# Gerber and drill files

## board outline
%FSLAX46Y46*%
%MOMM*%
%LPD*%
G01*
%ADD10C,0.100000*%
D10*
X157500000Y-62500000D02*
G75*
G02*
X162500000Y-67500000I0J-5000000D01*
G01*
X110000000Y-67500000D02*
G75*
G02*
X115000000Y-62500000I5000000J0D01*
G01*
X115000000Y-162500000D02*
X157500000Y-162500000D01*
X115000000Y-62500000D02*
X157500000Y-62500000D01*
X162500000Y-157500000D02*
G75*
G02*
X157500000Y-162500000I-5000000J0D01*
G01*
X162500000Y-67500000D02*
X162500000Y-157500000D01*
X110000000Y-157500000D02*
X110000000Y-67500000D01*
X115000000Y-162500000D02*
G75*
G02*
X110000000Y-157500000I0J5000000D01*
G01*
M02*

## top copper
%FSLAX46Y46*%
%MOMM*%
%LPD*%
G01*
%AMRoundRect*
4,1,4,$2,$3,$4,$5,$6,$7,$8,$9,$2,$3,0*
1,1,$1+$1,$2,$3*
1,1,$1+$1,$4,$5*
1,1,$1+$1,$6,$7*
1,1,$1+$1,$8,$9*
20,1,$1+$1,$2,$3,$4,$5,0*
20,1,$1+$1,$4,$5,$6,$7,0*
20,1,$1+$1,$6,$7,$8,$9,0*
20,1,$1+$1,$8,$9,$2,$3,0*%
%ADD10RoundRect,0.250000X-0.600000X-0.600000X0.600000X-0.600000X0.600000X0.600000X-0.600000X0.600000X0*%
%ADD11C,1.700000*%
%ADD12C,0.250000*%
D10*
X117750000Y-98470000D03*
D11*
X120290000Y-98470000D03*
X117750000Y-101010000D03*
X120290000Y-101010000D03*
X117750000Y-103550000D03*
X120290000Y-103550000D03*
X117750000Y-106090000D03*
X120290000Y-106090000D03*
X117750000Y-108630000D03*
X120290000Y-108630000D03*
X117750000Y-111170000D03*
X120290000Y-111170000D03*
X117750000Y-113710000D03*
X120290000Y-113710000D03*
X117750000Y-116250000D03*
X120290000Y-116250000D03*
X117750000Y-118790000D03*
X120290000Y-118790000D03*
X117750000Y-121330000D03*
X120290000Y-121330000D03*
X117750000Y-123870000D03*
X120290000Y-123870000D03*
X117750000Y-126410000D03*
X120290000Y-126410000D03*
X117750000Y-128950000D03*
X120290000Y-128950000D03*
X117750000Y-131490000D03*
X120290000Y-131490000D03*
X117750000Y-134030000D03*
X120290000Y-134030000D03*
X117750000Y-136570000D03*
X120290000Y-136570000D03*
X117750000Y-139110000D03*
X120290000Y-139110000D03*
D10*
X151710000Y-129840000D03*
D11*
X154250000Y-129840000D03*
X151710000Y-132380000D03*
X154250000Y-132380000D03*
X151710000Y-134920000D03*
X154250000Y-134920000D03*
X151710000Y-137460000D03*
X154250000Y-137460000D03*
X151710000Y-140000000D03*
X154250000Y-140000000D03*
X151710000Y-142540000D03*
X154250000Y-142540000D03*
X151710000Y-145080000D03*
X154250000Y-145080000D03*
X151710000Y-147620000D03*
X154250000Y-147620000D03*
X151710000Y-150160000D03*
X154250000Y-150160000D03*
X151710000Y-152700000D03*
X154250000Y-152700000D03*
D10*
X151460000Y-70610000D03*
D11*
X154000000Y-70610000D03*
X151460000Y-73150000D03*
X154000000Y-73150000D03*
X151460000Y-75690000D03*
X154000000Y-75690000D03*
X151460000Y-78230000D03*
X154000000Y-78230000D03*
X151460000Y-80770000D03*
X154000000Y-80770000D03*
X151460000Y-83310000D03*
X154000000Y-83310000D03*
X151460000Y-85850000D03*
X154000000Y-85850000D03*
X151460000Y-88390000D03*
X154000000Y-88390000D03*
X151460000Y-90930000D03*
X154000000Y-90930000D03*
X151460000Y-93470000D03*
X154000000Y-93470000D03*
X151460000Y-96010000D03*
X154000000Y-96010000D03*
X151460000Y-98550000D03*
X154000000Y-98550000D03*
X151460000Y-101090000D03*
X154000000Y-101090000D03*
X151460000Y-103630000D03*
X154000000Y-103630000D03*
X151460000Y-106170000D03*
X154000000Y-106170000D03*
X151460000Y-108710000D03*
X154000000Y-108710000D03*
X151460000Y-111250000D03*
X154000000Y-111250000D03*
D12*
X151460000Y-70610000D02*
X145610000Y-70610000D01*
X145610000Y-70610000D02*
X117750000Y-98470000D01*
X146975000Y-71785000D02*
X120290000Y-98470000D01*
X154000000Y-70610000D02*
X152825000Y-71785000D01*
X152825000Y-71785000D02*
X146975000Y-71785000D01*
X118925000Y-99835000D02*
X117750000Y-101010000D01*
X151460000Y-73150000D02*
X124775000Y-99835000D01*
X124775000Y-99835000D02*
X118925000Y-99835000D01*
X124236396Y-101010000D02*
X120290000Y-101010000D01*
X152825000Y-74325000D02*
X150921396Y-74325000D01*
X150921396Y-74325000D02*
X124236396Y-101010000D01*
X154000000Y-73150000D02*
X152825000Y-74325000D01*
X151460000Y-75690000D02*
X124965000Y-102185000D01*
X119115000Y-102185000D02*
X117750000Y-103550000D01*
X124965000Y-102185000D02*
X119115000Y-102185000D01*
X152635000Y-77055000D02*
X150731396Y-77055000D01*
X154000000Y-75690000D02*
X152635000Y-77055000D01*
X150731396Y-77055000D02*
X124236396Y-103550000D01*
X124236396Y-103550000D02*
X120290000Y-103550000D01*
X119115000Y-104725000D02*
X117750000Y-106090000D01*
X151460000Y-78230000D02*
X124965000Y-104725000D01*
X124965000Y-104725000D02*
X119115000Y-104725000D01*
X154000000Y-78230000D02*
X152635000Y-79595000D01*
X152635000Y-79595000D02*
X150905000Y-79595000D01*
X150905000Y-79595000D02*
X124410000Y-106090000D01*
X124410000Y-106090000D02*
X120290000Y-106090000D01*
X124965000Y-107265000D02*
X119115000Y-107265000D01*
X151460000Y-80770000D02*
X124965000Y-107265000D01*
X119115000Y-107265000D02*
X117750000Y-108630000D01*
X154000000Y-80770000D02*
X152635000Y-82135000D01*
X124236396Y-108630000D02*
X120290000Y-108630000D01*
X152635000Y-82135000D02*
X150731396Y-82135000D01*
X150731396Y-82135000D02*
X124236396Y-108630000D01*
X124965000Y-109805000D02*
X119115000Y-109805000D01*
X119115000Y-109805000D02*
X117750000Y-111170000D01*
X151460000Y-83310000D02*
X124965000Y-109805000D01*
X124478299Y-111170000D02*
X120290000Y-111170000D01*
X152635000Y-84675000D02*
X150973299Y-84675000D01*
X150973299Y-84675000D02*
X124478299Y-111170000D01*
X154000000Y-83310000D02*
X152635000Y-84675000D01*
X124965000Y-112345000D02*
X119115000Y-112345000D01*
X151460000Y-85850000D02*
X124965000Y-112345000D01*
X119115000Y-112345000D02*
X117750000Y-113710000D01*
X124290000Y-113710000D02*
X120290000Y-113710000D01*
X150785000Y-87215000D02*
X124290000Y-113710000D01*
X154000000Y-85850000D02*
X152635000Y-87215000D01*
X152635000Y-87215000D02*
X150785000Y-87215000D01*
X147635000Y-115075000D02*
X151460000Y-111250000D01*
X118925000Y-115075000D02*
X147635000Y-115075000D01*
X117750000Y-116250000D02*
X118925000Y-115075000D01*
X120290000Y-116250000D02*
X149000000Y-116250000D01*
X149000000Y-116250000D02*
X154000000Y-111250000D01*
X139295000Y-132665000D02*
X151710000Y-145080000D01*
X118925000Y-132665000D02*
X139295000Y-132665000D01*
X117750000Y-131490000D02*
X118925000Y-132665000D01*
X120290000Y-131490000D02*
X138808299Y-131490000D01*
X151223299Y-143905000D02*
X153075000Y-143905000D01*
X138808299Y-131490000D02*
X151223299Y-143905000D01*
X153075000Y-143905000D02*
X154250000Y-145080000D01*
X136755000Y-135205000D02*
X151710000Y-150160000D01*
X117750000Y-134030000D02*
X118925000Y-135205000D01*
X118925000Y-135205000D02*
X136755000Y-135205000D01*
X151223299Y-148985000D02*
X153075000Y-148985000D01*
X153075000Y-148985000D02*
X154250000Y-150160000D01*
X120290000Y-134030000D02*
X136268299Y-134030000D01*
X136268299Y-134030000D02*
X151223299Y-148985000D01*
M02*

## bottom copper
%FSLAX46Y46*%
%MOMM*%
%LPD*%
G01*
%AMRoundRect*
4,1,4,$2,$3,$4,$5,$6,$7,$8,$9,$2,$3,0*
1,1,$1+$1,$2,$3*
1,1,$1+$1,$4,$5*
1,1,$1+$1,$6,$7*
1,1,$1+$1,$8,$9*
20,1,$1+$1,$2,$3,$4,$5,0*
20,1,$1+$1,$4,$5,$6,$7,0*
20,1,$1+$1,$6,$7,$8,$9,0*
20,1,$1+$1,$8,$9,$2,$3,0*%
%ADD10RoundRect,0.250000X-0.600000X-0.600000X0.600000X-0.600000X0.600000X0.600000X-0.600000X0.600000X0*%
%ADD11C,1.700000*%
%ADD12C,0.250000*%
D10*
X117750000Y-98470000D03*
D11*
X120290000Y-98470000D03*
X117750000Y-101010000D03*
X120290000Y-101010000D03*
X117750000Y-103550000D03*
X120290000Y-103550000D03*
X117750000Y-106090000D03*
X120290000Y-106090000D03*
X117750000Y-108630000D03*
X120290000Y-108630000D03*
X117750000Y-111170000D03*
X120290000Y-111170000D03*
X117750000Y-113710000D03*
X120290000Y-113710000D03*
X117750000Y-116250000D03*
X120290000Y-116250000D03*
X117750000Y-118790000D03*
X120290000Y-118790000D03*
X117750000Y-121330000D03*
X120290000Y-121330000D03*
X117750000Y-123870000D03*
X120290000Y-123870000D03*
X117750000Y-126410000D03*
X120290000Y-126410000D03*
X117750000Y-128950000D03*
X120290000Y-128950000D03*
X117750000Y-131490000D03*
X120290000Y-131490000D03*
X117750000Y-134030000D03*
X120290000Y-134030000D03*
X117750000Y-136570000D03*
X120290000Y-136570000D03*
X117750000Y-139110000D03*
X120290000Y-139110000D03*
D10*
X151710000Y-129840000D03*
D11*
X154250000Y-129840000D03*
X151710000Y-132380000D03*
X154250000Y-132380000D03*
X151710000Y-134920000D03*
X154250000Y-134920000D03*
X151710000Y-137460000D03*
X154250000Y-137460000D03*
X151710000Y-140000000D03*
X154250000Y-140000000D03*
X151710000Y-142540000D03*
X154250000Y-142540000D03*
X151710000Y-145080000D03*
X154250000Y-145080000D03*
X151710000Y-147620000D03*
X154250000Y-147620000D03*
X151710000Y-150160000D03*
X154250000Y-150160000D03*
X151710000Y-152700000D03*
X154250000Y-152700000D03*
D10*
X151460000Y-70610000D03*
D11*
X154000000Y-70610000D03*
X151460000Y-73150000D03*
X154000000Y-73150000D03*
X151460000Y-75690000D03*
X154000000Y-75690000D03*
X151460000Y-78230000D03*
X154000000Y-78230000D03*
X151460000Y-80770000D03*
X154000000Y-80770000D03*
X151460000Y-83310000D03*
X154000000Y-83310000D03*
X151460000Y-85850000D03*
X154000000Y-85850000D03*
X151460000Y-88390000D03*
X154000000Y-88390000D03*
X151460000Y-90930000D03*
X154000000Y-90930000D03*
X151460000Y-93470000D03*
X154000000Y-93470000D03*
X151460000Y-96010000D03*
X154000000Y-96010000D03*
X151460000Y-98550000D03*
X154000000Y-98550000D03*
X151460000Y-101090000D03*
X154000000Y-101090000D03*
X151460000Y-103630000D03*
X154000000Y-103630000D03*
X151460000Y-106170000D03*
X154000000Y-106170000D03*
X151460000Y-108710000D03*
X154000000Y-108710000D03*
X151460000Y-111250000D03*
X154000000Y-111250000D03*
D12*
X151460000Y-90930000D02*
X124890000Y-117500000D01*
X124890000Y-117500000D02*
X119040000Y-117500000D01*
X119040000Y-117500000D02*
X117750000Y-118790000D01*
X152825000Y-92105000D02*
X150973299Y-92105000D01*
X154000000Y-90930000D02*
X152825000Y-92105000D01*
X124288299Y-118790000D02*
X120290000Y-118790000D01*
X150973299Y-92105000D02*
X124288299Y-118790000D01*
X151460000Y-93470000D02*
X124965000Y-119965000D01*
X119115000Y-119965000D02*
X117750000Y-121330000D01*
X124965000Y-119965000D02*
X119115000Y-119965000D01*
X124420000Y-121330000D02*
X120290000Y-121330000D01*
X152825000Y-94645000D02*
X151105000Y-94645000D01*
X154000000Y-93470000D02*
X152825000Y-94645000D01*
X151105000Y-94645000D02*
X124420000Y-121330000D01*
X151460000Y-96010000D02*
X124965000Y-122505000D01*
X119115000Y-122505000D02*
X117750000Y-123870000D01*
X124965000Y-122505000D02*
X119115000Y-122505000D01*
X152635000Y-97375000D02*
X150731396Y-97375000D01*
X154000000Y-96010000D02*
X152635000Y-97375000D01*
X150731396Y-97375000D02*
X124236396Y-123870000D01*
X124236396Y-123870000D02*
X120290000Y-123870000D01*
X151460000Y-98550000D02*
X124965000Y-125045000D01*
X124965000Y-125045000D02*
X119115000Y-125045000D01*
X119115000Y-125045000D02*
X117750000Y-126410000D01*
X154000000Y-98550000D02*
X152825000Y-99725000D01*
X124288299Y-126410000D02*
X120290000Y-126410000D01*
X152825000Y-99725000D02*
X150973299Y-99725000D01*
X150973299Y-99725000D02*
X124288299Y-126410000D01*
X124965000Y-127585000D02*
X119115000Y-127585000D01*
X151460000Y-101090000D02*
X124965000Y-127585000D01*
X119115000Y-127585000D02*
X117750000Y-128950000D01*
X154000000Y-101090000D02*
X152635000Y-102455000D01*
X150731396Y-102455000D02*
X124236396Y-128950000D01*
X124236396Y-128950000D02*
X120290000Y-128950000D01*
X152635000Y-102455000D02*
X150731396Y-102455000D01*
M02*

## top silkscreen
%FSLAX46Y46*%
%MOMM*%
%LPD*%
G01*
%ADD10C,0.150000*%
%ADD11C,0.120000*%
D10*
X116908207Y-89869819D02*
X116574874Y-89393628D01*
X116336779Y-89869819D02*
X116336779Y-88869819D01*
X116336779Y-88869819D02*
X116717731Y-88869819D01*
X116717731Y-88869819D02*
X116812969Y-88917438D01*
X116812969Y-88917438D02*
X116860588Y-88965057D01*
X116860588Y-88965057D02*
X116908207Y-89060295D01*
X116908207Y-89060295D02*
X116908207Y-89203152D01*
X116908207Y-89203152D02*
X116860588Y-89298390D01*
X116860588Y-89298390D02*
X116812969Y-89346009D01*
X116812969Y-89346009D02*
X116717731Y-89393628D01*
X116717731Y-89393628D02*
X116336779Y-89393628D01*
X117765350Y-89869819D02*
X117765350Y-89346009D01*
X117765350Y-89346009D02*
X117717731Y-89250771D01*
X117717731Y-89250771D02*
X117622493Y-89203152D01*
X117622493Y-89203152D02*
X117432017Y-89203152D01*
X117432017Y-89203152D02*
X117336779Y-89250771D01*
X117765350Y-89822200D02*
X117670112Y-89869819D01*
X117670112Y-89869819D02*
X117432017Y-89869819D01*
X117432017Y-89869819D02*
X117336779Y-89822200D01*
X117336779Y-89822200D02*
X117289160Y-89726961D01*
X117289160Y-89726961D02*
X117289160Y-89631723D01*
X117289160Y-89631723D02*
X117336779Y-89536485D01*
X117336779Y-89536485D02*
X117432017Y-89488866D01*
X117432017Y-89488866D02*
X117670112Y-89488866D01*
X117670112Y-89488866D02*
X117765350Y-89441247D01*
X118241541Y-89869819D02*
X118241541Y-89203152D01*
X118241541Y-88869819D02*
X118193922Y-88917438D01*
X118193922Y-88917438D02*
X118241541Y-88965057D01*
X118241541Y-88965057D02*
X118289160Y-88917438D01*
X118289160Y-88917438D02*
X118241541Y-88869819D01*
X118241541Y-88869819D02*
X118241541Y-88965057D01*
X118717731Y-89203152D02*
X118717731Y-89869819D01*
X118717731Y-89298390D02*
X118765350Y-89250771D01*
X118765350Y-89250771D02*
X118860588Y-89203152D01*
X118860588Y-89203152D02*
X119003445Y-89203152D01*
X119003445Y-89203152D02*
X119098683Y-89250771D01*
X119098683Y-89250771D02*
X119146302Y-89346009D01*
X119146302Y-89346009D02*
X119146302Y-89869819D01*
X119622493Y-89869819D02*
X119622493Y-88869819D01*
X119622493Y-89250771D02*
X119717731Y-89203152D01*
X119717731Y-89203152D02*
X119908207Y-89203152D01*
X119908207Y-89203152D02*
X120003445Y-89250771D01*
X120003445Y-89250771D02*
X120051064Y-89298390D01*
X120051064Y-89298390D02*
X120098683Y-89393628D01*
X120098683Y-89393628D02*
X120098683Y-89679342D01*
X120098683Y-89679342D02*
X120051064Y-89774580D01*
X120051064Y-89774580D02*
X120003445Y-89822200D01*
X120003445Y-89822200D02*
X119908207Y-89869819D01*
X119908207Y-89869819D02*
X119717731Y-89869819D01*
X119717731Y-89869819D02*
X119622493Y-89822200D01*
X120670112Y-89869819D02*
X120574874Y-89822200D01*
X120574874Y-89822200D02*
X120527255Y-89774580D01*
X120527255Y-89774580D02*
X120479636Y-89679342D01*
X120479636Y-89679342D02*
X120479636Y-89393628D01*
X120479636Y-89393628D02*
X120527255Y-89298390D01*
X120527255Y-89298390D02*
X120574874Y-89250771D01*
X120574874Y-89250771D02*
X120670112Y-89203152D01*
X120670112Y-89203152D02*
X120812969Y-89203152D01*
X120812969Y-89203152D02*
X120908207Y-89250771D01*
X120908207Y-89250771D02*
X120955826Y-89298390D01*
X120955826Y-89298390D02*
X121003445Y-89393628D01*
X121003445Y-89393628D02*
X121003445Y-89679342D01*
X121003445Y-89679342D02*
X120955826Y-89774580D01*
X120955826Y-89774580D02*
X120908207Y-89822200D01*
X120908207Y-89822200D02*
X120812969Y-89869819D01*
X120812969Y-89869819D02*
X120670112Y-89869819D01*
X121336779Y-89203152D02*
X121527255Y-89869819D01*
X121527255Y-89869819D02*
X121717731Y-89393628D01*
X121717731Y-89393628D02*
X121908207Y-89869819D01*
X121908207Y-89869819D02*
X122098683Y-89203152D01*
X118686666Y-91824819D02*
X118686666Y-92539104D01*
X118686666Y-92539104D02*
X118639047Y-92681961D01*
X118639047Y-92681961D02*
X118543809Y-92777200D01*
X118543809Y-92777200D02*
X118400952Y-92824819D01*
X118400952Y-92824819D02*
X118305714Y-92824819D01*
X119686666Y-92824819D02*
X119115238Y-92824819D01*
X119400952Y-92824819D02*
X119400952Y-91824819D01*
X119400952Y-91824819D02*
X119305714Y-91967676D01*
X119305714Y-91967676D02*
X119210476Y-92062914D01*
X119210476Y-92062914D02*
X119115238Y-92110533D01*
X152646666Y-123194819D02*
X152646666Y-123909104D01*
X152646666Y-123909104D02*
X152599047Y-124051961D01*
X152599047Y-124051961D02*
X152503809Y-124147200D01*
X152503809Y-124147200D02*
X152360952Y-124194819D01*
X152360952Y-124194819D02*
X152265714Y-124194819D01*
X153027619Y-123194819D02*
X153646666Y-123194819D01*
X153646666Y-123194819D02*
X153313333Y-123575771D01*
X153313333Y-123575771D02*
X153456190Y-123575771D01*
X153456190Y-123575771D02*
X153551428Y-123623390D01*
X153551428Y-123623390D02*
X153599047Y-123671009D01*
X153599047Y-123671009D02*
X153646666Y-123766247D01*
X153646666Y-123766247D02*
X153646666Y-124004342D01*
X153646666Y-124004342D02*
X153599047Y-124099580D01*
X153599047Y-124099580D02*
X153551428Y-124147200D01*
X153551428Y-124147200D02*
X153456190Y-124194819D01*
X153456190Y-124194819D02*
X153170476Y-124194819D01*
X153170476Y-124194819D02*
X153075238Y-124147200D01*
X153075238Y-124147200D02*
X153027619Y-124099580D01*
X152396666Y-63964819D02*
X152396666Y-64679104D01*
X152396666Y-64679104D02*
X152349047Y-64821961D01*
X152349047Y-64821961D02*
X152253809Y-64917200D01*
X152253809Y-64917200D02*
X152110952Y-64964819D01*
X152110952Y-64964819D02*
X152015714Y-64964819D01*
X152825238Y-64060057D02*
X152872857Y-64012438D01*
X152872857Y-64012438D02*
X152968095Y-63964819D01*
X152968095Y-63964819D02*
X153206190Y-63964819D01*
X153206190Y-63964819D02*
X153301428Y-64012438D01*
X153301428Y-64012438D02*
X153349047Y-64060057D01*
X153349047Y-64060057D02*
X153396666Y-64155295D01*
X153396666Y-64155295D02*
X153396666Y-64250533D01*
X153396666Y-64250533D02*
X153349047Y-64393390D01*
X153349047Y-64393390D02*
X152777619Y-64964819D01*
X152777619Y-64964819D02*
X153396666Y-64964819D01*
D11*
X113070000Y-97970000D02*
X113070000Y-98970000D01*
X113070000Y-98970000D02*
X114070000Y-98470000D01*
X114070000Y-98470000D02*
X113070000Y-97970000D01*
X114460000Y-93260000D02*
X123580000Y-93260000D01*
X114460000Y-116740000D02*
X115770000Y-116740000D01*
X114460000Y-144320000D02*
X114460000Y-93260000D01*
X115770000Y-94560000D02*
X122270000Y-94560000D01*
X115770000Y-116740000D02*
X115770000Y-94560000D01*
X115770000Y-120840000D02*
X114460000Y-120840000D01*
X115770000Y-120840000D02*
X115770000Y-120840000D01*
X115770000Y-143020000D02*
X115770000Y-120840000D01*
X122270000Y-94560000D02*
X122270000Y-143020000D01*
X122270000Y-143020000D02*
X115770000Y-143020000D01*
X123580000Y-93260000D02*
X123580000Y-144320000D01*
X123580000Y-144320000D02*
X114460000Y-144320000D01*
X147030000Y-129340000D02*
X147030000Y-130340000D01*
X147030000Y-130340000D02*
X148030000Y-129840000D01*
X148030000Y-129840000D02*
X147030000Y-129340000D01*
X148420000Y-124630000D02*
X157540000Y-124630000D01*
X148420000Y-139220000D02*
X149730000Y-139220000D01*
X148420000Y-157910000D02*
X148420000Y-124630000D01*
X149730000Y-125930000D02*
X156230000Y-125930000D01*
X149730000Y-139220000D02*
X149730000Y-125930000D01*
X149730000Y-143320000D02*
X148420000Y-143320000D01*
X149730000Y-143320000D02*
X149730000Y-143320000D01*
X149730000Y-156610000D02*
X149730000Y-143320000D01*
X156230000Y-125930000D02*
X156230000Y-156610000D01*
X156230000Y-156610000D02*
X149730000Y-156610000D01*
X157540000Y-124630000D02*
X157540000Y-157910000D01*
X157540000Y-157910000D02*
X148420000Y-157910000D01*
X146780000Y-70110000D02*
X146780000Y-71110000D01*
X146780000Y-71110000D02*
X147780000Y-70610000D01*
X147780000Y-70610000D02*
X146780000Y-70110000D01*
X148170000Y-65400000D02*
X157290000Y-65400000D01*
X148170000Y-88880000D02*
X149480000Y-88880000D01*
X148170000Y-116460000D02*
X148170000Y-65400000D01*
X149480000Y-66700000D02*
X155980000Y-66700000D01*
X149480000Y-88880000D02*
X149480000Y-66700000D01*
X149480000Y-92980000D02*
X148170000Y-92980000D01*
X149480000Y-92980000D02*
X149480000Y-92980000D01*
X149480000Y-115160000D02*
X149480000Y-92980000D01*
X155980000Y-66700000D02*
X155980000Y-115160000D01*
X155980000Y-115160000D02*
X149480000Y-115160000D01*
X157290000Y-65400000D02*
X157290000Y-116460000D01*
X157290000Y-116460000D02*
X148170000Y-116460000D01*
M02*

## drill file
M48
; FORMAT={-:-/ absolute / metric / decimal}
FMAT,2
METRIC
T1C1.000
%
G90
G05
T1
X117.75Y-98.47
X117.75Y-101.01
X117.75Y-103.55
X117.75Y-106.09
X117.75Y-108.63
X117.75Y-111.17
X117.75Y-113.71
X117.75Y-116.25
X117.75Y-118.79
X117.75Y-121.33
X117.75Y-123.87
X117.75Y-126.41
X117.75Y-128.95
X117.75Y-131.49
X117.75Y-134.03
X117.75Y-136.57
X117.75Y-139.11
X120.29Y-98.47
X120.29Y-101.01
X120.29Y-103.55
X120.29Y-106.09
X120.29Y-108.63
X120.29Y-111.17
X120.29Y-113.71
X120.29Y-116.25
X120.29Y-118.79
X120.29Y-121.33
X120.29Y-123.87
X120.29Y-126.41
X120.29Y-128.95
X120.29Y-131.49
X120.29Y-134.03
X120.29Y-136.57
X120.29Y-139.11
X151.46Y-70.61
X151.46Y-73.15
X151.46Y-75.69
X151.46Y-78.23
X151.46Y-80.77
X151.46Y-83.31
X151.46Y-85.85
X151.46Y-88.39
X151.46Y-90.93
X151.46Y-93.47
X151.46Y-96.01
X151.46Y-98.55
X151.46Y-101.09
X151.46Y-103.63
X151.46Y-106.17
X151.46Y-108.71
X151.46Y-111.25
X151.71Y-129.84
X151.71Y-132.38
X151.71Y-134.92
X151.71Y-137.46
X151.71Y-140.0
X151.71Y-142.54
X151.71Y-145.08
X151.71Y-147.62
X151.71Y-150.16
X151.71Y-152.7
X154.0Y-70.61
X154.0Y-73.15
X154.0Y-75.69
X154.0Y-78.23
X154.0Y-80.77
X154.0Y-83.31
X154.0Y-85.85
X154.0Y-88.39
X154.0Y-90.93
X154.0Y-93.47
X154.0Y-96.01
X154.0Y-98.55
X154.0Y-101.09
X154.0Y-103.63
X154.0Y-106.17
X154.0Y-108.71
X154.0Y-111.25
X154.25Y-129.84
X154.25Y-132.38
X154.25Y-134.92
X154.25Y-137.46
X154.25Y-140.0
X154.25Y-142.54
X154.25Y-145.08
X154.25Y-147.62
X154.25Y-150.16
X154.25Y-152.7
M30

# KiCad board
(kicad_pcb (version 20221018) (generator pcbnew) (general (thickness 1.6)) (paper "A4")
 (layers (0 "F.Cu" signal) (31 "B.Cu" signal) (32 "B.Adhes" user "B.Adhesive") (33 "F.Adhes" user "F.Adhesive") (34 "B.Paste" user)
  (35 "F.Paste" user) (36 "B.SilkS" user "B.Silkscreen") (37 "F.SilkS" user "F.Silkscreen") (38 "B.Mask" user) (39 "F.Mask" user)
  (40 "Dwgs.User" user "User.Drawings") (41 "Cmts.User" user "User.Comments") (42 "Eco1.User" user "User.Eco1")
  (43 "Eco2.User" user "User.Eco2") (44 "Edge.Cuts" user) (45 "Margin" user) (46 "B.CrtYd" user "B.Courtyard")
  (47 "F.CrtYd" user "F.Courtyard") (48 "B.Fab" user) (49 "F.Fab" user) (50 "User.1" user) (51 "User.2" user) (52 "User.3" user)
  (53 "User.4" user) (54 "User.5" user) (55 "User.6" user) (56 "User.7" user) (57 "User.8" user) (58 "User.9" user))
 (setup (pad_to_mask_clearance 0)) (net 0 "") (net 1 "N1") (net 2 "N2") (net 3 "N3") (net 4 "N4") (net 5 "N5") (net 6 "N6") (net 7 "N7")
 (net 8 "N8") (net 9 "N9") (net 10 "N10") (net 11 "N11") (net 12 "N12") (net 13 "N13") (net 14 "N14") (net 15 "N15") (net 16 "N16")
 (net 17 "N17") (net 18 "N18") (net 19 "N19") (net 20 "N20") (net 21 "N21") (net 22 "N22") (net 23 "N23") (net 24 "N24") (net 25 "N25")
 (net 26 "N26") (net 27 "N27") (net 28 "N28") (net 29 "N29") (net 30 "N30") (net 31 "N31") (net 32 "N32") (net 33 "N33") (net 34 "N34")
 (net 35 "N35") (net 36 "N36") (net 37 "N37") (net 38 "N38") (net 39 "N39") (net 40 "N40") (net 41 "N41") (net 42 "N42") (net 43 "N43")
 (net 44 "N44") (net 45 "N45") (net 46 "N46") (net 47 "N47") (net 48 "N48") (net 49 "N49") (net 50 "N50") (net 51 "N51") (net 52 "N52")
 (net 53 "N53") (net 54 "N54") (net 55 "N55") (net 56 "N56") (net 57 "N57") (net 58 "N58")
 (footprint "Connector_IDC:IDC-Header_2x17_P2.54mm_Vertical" (layer "F.Cu") (at 117.75 98.47)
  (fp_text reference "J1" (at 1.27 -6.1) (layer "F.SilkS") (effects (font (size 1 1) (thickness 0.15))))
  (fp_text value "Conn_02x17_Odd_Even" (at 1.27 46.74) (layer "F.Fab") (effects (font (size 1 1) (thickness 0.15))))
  (fp_line (start -4.68 -0.5) (end -4.68 0.5) (stroke (width 0.12) (type solid)) (layer "F.SilkS"))
  (fp_line (start -4.68 0.5) (end -3.68 0) (stroke (width 0.12) (type solid)) (layer "F.SilkS"))
  (fp_line (start -3.68 0) (end -4.68 -0.5) (stroke (width 0.12) (type solid)) (layer "F.SilkS"))
  (fp_line (start -3.29 -5.21) (end 5.83 -5.21) (stroke (width 0.12) (type solid)) (layer "F.SilkS"))
  (fp_line (start -3.29 18.27) (end -1.98 18.27) (stroke (width 0.12) (type solid)) (layer "F.SilkS"))
  (fp_line (start -3.29 45.85) (end -3.29 -5.21) (stroke (width 0.12) (type solid)) (layer "F.SilkS"))
  (fp_line (start -1.98 -3.91) (end 4.52 -3.91) (stroke (width 0.12) (type solid)) (layer "F.SilkS"))
  (fp_line (start -1.98 18.27) (end -1.98 -3.91) (stroke (width 0.12) (type solid)) (layer "F.SilkS"))
  (fp_line (start -1.98 22.37) (end -3.29 22.37) (stroke (width 0.12) (type solid)) (layer "F.SilkS"))
  (fp_line (start -1.98 22.37) (end -1.98 22.37) (stroke (width 0.12) (type solid)) (layer "F.SilkS"))
  (fp_line (start -1.98 44.55) (end -1.98 22.37) (stroke (width 0.12) (type solid)) (layer "F.SilkS"))
  (fp_line (start 4.52 -3.91) (end 4.52 44.55) (stroke (width 0.12) (type solid)) (layer "F.SilkS"))
  (fp_line (start 4.52 44.55) (end -1.98 44.55) (stroke (width 0.12) (type solid)) (layer "F.SilkS"))
  (fp_line (start 5.83 -5.21) (end 5.83 45.85) (stroke (width 0.12) (type solid)) (layer "F.SilkS"))
  (fp_line (start 5.83 45.85) (end -3.29 45.85) (stroke (width 0.12) (type solid)) (layer "F.SilkS"))
  (pad "1" thru_hole roundrect (at 0 0) (size 1.7 1.7) (drill 1) (layers "*.Cu" "*.Mask") (roundrect_rratio 0.1470588235) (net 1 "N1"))
  (pad "2" thru_hole circle (at 2.54 0) (size 1.7 1.7) (drill 1) (layers "*.Cu" "*.Mask") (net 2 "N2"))
  (pad "3" thru_hole circle (at 0 2.54) (size 1.7 1.7) (drill 1) (layers "*.Cu" "*.Mask") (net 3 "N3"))
  (pad "4" thru_hole circle (at 2.54 2.54) (size 1.7 1.7) (drill 1) (layers "*.Cu" "*.Mask") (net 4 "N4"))
  (pad "5" thru_hole circle (at 0 5.08) (size 1.7 1.7) (drill 1) (layers "*.Cu" "*.Mask") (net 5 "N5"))
  (pad "6" thru_hole circle (at 2.54 5.08) (size 1.7 1.7) (drill 1) (layers "*.Cu" "*.Mask") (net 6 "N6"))
  (pad "7" thru_hole circle (at 0 7.62) (size 1.7 1.7) (drill 1) (layers "*.Cu" "*.Mask") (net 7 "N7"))
  (pad "8" thru_hole circle (at 2.54 7.62) (size 1.7 1.7) (drill 1) (layers "*.Cu" "*.Mask") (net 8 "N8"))
  (pad "9" thru_hole circle (at 0 10.16) (size 1.7 1.7) (drill 1) (layers "*.Cu" "*.Mask") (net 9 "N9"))
  (pad "10" thru_hole circle (at 2.54 10.16) (size 1.7 1.7) (drill 1) (layers "*.Cu" "*.Mask") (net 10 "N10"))
  (pad "11" thru_hole circle (at 0 12.7) (size 1.7 1.7) (drill 1) (layers "*.Cu" "*.Mask") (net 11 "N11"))
  (pad "12" thru_hole circle (at 2.54 12.7) (size 1.7 1.7) (drill 1) (layers "*.Cu" "*.Mask") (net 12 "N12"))
  (pad "13" thru_hole circle (at 0 15.24) (size 1.7 1.7) (drill 1) (layers "*.Cu" "*.Mask") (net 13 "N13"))
  (pad "14" thru_hole circle (at 2.54 15.24) (size 1.7 1.7) (drill 1) (layers "*.Cu" "*.Mask") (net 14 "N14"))
  (pad "15" thru_hole circle (at 0 17.78) (size 1.7 1.7) (drill 1) (layers "*.Cu" "*.Mask") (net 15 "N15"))
  (pad "16" thru_hole circle (at 2.54 17.78) (size 1.7 1.7) (drill 1) (layers "*.Cu" "*.Mask") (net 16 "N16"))
  (pad "17" thru_hole circle (at 0 20.32) (size 1.7 1.7) (drill 1) (layers "*.Cu" "*.Mask") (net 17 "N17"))
  (pad "18" thru_hole circle (at 2.54 20.32) (size 1.7 1.7) (drill 1) (layers "*.Cu" "*.Mask") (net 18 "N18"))
  (pad "19" thru_hole circle (at 0 22.86) (size 1.7 1.7) (drill 1) (layers "*.Cu" "*.Mask") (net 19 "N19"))
  (pad "20" thru_hole circle (at 2.54 22.86) (size 1.7 1.7) (drill 1) (layers "*.Cu" "*.Mask") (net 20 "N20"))
  (pad "21" thru_hole circle (at 0 25.4) (size 1.7 1.7) (drill 1) (layers "*.Cu" "*.Mask") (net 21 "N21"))
  (pad "22" thru_hole circle (at 2.54 25.4) (size 1.7 1.7) (drill 1) (layers "*.Cu" "*.Mask") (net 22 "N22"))
  (pad "23" thru_hole circle (at 0 27.94) (size 1.7 1.7) (drill 1) (layers "*.Cu" "*.Mask") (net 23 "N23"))
  (pad "24" thru_hole circle (at 2.54 27.94) (size 1.7 1.7) (drill 1) (layers "*.Cu" "*.Mask") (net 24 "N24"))
  (pad "25" thru_hole circle (at 0 30.48) (size 1.7 1.7) (drill 1) (layers "*.Cu" "*.Mask") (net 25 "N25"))
  (pad "26" thru_hole circle (at 2.54 30.48) (size 1.7 1.7) (drill 1) (layers "*.Cu" "*.Mask") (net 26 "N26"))
  (pad "27" thru_hole circle (at 0 33.02) (size 1.7 1.7) (drill 1) (layers "*.Cu" "*.Mask") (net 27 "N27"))
  (pad "28" thru_hole circle (at 2.54 33.02) (size 1.7 1.7) (drill 1) (layers "*.Cu" "*.Mask") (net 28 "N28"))
  (pad "29" thru_hole circle (at 0 35.56) (size 1.7 1.7) (drill 1) (layers "*.Cu" "*.Mask") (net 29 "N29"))
  (pad "30" thru_hole circle (at 2.54 35.56) (size 1.7 1.7) (drill 1) (layers "*.Cu" "*.Mask") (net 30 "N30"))
  (pad "31" thru_hole circle (at 0 38.1) (size 1.7 1.7) (drill 1) (layers "*.Cu" "*.Mask") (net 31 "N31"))
  (pad "32" thru_hole circle (at 2.54 38.1) (size 1.7 1.7) (drill 1) (layers "*.Cu" "*.Mask") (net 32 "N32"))
  (pad "33" thru_hole circle (at 0 40.64) (size 1.7 1.7) (drill 1) (layers "*.Cu" "*.Mask") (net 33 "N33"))
  (pad "34" thru_hole circle (at 2.54 40.64) (size 1.7 1.7) (drill 1) (layers "*.Cu" "*.Mask") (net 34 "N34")))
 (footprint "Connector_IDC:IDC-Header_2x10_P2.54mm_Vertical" (layer "F.Cu") (at 151.71 129.84)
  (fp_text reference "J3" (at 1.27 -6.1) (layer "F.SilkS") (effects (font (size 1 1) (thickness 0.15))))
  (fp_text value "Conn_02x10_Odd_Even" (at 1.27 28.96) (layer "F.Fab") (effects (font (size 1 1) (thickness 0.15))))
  (fp_line (start -4.68 -0.5) (end -4.68 0.5) (stroke (width 0.12) (type solid)) (layer "F.SilkS"))
  (fp_line (start -4.68 0.5) (end -3.68 0) (stroke (width 0.12) (type solid)) (layer "F.SilkS"))
  (fp_line (start -3.68 0) (end -4.68 -0.5) (stroke (width 0.12) (type solid)) (layer "F.SilkS"))
  (fp_line (start -3.29 -5.21) (end 5.83 -5.21) (stroke (width 0.12) (type solid)) (layer "F.SilkS"))
  (fp_line (start -3.29 9.38) (end -1.98 9.38) (stroke (width 0.12) (type solid)) (layer "F.SilkS"))
  (fp_line (start -3.29 28.07) (end -3.29 -5.21) (stroke (width 0.12) (type solid)) (layer "F.SilkS"))
  (fp_line (start -1.98 -3.91) (end 4.52 -3.91) (stroke (width 0.12) (type solid)) (layer "F.SilkS"))
  (fp_line (start -1.98 9.38) (end -1.98 -3.91) (stroke (width 0.12) (type solid)) (layer "F.SilkS"))
  (fp_line (start -1.98 13.48) (end -3.29 13.48) (stroke (width 0.12) (type solid)) (layer "F.SilkS"))
  (fp_line (start -1.98 13.48) (end -1.98 13.48) (stroke (width 0.12) (type solid)) (layer "F.SilkS"))
  (fp_line (start -1.98 26.77) (end -1.98 13.48) (stroke (width 0.12) (type solid)) (layer "F.SilkS"))
  (fp_line (start 4.52 -3.91) (end 4.52 26.77) (stroke (width 0.12) (type solid)) (layer "F.SilkS"))
  (fp_line (start 4.52 26.77) (end -1.98 26.77) (stroke (width 0.12) (type solid)) (layer "F.SilkS"))
  (fp_line (start 5.83 -5.21) (end 5.83 28.07) (stroke (width 0.12) (type solid)) (layer "F.SilkS"))
  (fp_line (start 5.83 28.07) (end -3.29 28.07) (stroke (width 0.12) (type solid)) (layer "F.SilkS"))
  (pad "1" thru_hole roundrect (at 0 0) (size 1.7 1.7) (drill 1) (layers "*.Cu" "*.Mask") (roundrect_rratio 0.1470588235) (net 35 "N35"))
  (pad "2" thru_hole circle (at 2.54 0) (size 1.7 1.7) (drill 1) (layers "*.Cu" "*.Mask") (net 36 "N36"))
  (pad "3" thru_hole circle (at 0 2.54) (size 1.7 1.7) (drill 1) (layers "*.Cu" "*.Mask") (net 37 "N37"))
  (pad "4" thru_hole circle (at 2.54 2.54) (size 1.7 1.7) (drill 1) (layers "*.Cu" "*.Mask") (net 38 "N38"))
  (pad "5" thru_hole circle (at 0 5.08) (size 1.7 1.7) (drill 1) (layers "*.Cu" "*.Mask") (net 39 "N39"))
  (pad "6" thru_hole circle (at 2.54 5.08) (size 1.7 1.7) (drill 1) (layers "*.Cu" "*.Mask") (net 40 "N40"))
  (pad "7" thru_hole circle (at 0 7.62) (size 1.7 1.7) (drill 1) (layers "*.Cu" "*.Mask") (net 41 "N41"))
  (pad "8" thru_hole circle (at 2.54 7.62) (size 1.7 1.7) (drill 1) (layers "*.Cu" "*.Mask") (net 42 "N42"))
  (pad "9" thru_hole circle (at 0 10.16) (size 1.7 1.7) (drill 1) (layers "*.Cu" "*.Mask") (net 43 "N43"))
  (pad "10" thru_hole circle (at 2.54 10.16) (size 1.7 1.7) (drill 1) (layers "*.Cu" "*.Mask") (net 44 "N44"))
  (pad "11" thru_hole circle (at 0 12.7) (size 1.7 1.7) (drill 1) (layers "*.Cu" "*.Mask") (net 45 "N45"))
  (pad "12" thru_hole circle (at 2.54 12.7) (size 1.7 1.7) (drill 1) (layers "*.Cu" "*.Mask") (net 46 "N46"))
  (pad "13" thru_hole circle (at 0 15.24) (size 1.7 1.7) (drill 1) (layers "*.Cu" "*.Mask") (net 27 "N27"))
  (pad "14" thru_hole circle (at 2.54 15.24) (size 1.7 1.7) (drill 1) (layers "*.Cu" "*.Mask") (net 28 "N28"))
  (pad "15" thru_hole circle (at 0 17.78) (size 1.7 1.7) (drill 1) (layers "*.Cu" "*.Mask") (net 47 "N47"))
  (pad "16" thru_hole circle (at 2.54 17.78) (size 1.7 1.7) (drill 1) (layers "*.Cu" "*.Mask") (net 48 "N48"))
  (pad "17" thru_hole circle (at 0 20.32) (size 1.7 1.7) (drill 1) (layers "*.Cu" "*.Mask") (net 29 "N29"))
  (pad "18" thru_hole circle (at 2.54 20.32) (size 1.7 1.7) (drill 1) (layers "*.Cu" "*.Mask") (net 30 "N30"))
  (pad "19" thru_hole circle (at 0 22.86) (size 1.7 1.7) (drill 1) (layers "*.Cu" "*.Mask") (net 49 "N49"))
  (pad "20" thru_hole circle (at 2.54 22.86) (size 1.7 1.7) (drill 1) (layers "*.Cu" "*.Mask") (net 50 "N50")))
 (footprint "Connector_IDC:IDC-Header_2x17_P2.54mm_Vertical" (layer "F.Cu") (at 151.46 70.61)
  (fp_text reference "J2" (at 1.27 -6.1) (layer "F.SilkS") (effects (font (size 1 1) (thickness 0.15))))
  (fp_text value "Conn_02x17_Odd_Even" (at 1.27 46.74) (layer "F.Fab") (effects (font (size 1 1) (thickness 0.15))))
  (fp_line (start -4.68 -0.5) (end -4.68 0.5) (stroke (width 0.12) (type solid)) (layer "F.SilkS"))
  (fp_line (start -4.68 0.5) (end -3.68 0) (stroke (width 0.12) (type solid)) (layer "F.SilkS"))
  (fp_line (start -3.68 0) (end -4.68 -0.5) (stroke (width 0.12) (type solid)) (layer "F.SilkS"))
  (fp_line (start -3.29 -5.21) (end 5.83 -5.21) (stroke (width 0.12) (type solid)) (layer "F.SilkS"))
  (fp_line (start -3.29 18.27) (end -1.98 18.27) (stroke (width 0.12) (type solid)) (layer "F.SilkS"))
  (fp_line (start -3.29 45.85) (end -3.29 -5.21) (stroke (width 0.12) (type solid)) (layer "F.SilkS"))
  (fp_line (start -1.98 -3.91) (end 4.52 -3.91) (stroke (width 0.12) (type solid)) (layer "F.SilkS"))
  (fp_line (start -1.98 18.27) (end -1.98 -3.91) (stroke (width 0.12) (type solid)) (layer "F.SilkS"))
  (fp_line (start -1.98 22.37) (end -3.29 22.37) (stroke (width 0.12) (type solid)) (layer "F.SilkS"))
  (fp_line (start -1.98 22.37) (end -1.98 22.37) (stroke (width 0.12) (type solid)) (layer "F.SilkS"))
  (fp_line (start -1.98 44.55) (end -1.98 22.37) (stroke (width 0.12) (type solid)) (layer "F.SilkS"))
  (fp_line (start 4.52 -3.91) (end 4.52 44.55) (stroke (width 0.12) (type solid)) (layer "F.SilkS"))
  (fp_line (start 4.52 44.55) (end -1.98 44.55) (stroke (width 0.12) (type solid)) (layer "F.SilkS"))
  (fp_line (start 5.83 -5.21) (end 5.83 45.85) (stroke (width 0.12) (type solid)) (layer "F.SilkS"))
  (fp_line (start 5.83 45.85) (end -3.29 45.85) (stroke (width 0.12) (type solid)) (layer "F.SilkS"))
  (pad "1" thru_hole roundrect (at 0 0) (size 1.7 1.7) (drill 1) (layers "*.Cu" "*.Mask") (roundrect_rratio 0.1470588235) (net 1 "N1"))
  (pad "2" thru_hole circle (at 2.54 0) (size 1.7 1.7) (drill 1) (layers "*.Cu" "*.Mask") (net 2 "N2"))
  (pad "3" thru_hole circle (at 0 2.54) (size 1.7 1.7) (drill 1) (layers "*.Cu" "*.Mask") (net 3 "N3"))
  (pad "4" thru_hole circle (at 2.54 2.54) (size 1.7 1.7) (drill 1) (layers "*.Cu" "*.Mask") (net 4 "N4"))
  (pad "5" thru_hole circle (at 0 5.08) (size 1.7 1.7) (drill 1) (layers "*.Cu" "*.Mask") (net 5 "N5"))
  (pad "6" thru_hole circle (at 2.54 5.08) (size 1.7 1.7) (drill 1) (layers "*.Cu" "*.Mask") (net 6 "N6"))
  (pad "7" thru_hole circle (at 0 7.62) (size 1.7 1.7) (drill 1) (layers "*.Cu" "*.Mask") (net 7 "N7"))
  (pad "8" thru_hole circle (at 2.54 7.62) (size 1.7 1.7) (drill 1) (layers "*.Cu" "*.Mask") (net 8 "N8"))
  (pad "9" thru_hole circle (at 0 10.16) (size 1.7 1.7) (drill 1) (layers "*.Cu" "*.Mask") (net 9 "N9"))
  (pad "10" thru_hole circle (at 2.54 10.16) (size 1.7 1.7) (drill 1) (layers "*.Cu" "*.Mask") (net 10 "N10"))
  (pad "11" thru_hole circle (at 0 12.7) (size 1.7 1.7) (drill 1) (layers "*.Cu" "*.Mask") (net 11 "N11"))
  (pad "12" thru_hole circle (at 2.54 12.7) (size 1.7 1.7) (drill 1) (layers "*.Cu" "*.Mask") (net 12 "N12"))
  (pad "13" thru_hole circle (at 0 15.24) (size 1.7 1.7) (drill 1) (layers "*.Cu" "*.Mask") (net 13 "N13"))
  (pad "14" thru_hole circle (at 2.54 15.24) (size 1.7 1.7) (drill 1) (layers "*.Cu" "*.Mask") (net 14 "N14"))
  (pad "15" thru_hole circle (at 0 17.78) (size 1.7 1.7) (drill 1) (layers "*.Cu" "*.Mask") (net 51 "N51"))
  (pad "16" thru_hole circle (at 2.54 17.78) (size 1.7 1.7) (drill 1) (layers "*.Cu" "*.Mask") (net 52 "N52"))
  (pad "17" thru_hole circle (at 0 20.32) (size 1.7 1.7) (drill 1) (layers "*.Cu" "*.Mask") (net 17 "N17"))
  (pad "18" thru_hole circle (at 2.54 20.32) (size 1.7 1.7) (drill 1) (layers "*.Cu" "*.Mask") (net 18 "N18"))
  (pad "19" thru_hole circle (at 0 22.86) (size 1.7 1.7) (drill 1) (layers "*.Cu" "*.Mask") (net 19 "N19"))
  (pad "20" thru_hole circle (at 2.54 22.86) (size 1.7 1.7) (drill 1) (layers "*.Cu" "*.Mask") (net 20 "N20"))
  (pad "21" thru_hole circle (at 0 25.4) (size 1.7 1.7) (drill 1) (layers "*.Cu" "*.Mask") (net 21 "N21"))
  (pad "22" thru_hole circle (at 2.54 25.4) (size 1.7 1.7) (drill 1) (layers "*.Cu" "*.Mask") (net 22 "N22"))
  (pad "23" thru_hole circle (at 0 27.94) (size 1.7 1.7) (drill 1) (layers "*.Cu" "*.Mask") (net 23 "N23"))
  (pad "24" thru_hole circle (at 2.54 27.94) (size 1.7 1.7) (drill 1) (layers "*.Cu" "*.Mask") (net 24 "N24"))
  (pad "25" thru_hole circle (at 0 30.48) (size 1.7 1.7) (drill 1) (layers "*.Cu" "*.Mask") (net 25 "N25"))
  (pad "26" thru_hole circle (at 2.54 30.48) (size 1.7 1.7) (drill 1) (layers "*.Cu" "*.Mask") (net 26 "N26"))
  (pad "27" thru_hole circle (at 0 33.02) (size 1.7 1.7) (drill 1) (layers "*.Cu" "*.Mask") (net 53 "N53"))
  (pad "28" thru_hole circle (at 2.54 33.02) (size 1.7 1.7) (drill 1) (layers "*.Cu" "*.Mask") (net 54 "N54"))
  (pad "29" thru_hole circle (at 0 35.56) (size 1.7 1.7) (drill 1) (layers "*.Cu" "*.Mask") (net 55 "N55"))
  (pad "30" thru_hole circle (at 2.54 35.56) (size 1.7 1.7) (drill 1) (layers "*.Cu" "*.Mask") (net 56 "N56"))
  (pad "31" thru_hole circle (at 0 38.1) (size 1.7 1.7) (drill 1) (layers "*.Cu" "*.Mask") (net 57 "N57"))
  (pad "32" thru_hole circle (at 2.54 38.1) (size 1.7 1.7) (drill 1) (layers "*.Cu" "*.Mask") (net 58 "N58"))
  (pad "33" thru_hole circle (at 0 40.64) (size 1.7 1.7) (drill 1) (layers "*.Cu" "*.Mask") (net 15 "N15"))
  (pad "34" thru_hole circle (at 2.54 40.64) (size 1.7 1.7) (drill 1) (layers "*.Cu" "*.Mask") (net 16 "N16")))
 (gr_arc (start 157.5 62.5) (mid 161.035534 63.964466) (end 162.5 67.5) (stroke (width 0.1) (type default)) (layer "Edge.Cuts"))
 (gr_arc (start 110 67.5) (mid 111.464466 63.964466) (end 115 62.5) (stroke (width 0.1) (type default)) (layer "Edge.Cuts"))
 (gr_line (start 115 162.5) (end 157.5 162.5) (stroke (width 0.1) (type default)) (layer "Edge.Cuts"))
 (gr_line (start 115 62.5) (end 157.5 62.5) (stroke (width 0.1) (type default)) (layer "Edge.Cuts"))
 (gr_arc (start 162.5 157.5) (mid 161.035534 161.035534) (end 157.5 162.5) (stroke (width 0.1) (type default)) (layer "Edge.Cuts"))
 (gr_line (start 162.5 67.5) (end 162.5 157.5) (stroke (width 0.1) (type default)) (layer "Edge.Cuts"))
 (gr_line (start 110 157.5) (end 110 67.5) (stroke (width 0.1) (type default)) (layer "Edge.Cuts"))
 (gr_arc (start 115 162.5) (mid 111.464466 161.035534) (end 110 157.5) (stroke (width 0.1) (type default)) (layer "Edge.Cuts"))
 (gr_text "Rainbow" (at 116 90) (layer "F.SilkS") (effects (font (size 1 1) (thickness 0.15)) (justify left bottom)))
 (segment (start 151.46 70.61) (end 145.61 70.61) (width 0.25) (layer "F.Cu") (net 1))
 (segment (start 145.61 70.61) (end 117.75 98.47) (width 0.25) (layer "F.Cu") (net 1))
 (segment (start 146.975 71.785) (end 120.29 98.47) (width 0.25) (layer "F.Cu") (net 2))
 (segment (start 154 70.61) (end 152.825 71.785) (width 0.25) (layer "F.Cu") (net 2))
 (segment (start 152.825 71.785) (end 146.975 71.785) (width 0.25) (layer "F.Cu") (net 2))
 (segment (start 118.925 99.835) (end 117.75 101.01) (width 0.25) (layer "F.Cu") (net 3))
 (segment (start 151.46 73.15) (end 124.775 99.835) (width 0.25) (layer "F.Cu") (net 3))
 (segment (start 124.775 99.835) (end 118.925 99.835) (width 0.25) (layer "F.Cu") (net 3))
 (segment (start 124.236396 101.01) (end 120.29 101.01) (width 0.25) (layer "F.Cu") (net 4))
 (segment (start 152.825 74.325) (end 150.921396 74.325) (width 0.25) (layer "F.Cu") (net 4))
 (segment (start 150.921396 74.325) (end 124.236396 101.01) (width 0.25) (layer "F.Cu") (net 4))
 (segment (start 154 73.15) (end 152.825 74.325) (width 0.25) (layer "F.Cu") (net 4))
 (segment (start 151.46 75.69) (end 124.965 102.185) (width 0.25) (layer "F.Cu") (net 5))
 (segment (start 119.115 102.185) (end 117.75 103.55) (width 0.25) (layer "F.Cu") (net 5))
 (segment (start 124.965 102.185) (end 119.115 102.185) (width 0.25) (layer "F.Cu") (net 5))
 (segment (start 152.635 77.055) (end 150.731396 77.055) (width 0.25) (layer "F.Cu") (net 6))
 (segment (start 154 75.69) (end 152.635 77.055) (width 0.25) (layer "F.Cu") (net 6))
 (segment (start 150.731396 77.055) (end 124.236396 103.55) (width 0.25) (layer "F.Cu") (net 6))
 (segment (start 124.236396 103.55) (end 120.29 103.55) (width 0.25) (layer "F.Cu") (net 6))
 (segment (start 119.115 104.725) (end 117.75 106.09) (width 0.25) (layer "F.Cu") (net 7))
 (segment (start 151.46 78.23) (end 124.965 104.725) (width 0.25) (layer "F.Cu") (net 7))
 (segment (start 124.965 104.725) (end 119.115 104.725) (width 0.25) (layer "F.Cu") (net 7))
 (segment (start 154 78.23) (end 152.635 79.595) (width 0.25) (layer "F.Cu") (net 8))
 (segment (start 152.635 79.595) (end 150.905 79.595) (width 0.25) (layer "F.Cu") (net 8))
 (segment (start 150.905 79.595) (end 124.41 106.09) (width 0.25) (layer "F.Cu") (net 8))
 (segment (start 124.41 106.09) (end 120.29 106.09) (width 0.25) (layer "F.Cu") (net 8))
 (segment (start 124.965 107.265) (end 119.115 107.265) (width 0.25) (layer "F.Cu") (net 9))
 (segment (start 151.46 80.77) (end 124.965 107.265) (width 0.25) (layer "F.Cu") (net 9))
 (segment (start 119.115 107.265) (end 117.75 108.63) (width 0.25) (layer "F.Cu") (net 9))
 (segment (start 154 80.77) (end 152.635 82.135) (width 0.25) (layer "F.Cu") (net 10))
 (segment (start 124.236396 108.63) (end 120.29 108.63) (width 0.25) (layer "F.Cu") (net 10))
 (segment (start 152.635 82.135) (end 150.731396 82.135) (width 0.25) (layer "F.Cu") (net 10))
 (segment (start 150.731396 82.135) (end 124.236396 108.63) (width 0.25) (layer "F.Cu") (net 10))
 (segment (start 124.965 109.805) (end 119.115 109.805) (width 0.25) (layer "F.Cu") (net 11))
 (segment (start 119.115 109.805) (end 117.75 111.17) (width 0.25) (layer "F.Cu") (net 11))
 (segment (start 151.46 83.31) (end 124.965 109.805) (width 0.25) (layer "F.Cu") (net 11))
 (segment (start 124.478299 111.17) (end 120.29 111.17) (width 0.25) (layer "F.Cu") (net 12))
 (segment (start 152.635 84.675) (end 150.973299 84.675) (width 0.25) (layer "F.Cu") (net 12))
 (segment (start 150.973299 84.675) (end 124.478299 111.17) (width 0.25) (layer "F.Cu") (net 12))
 (segment (start 154 83.31) (end 152.635 84.675) (width 0.25) (layer "F.Cu") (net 12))
 (segment (start 124.965 112.345) (end 119.115 112.345) (width 0.25) (layer "F.Cu") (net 13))
 (segment (start 151.46 85.85) (end 124.965 112.345) (width 0.25) (layer "F.Cu") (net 13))
 (segment (start 119.115 112.345) (end 117.75 113.71) (width 0.25) (layer "F.Cu") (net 13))
 (segment (start 124.29 113.71) (end 120.29 113.71) (width 0.25) (layer "F.Cu") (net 14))
 (segment (start 150.785 87.215) (end 124.29 113.71) (width 0.25) (layer "F.Cu") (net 14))
 (segment (start 154 85.85) (end 152.635 87.215) (width 0.25) (layer "F.Cu") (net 14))
 (segment (start 152.635 87.215) (end 150.785 87.215) (width 0.25) (layer "F.Cu") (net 14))
 (segment (start 147.635 115.075) (end 151.46 111.25) (width 0.25) (layer "F.Cu") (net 15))
 (segment (start 118.925 115.075) (end 147.635 115.075) (width 0.25) (layer "F.Cu") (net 15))
 (segment (start 117.75 116.25) (end 118.925 115.075) (width 0.25) (layer "F.Cu") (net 15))
 (segment (start 120.29 116.25) (end 149 116.25) (width 0.25) (layer "F.Cu") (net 16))
 (segment (start 149 116.25) (end 154 111.25) (width 0.25) (layer "F.Cu") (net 16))
 (segment (start 151.46 90.93) (end 124.89 117.5) (width 0.25) (layer "B.Cu") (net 17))
 (segment (start 124.89 117.5) (end 119.04 117.5) (width 0.25) (layer "B.Cu") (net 17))
 (segment (start 119.04 117.5) (end 117.75 118.79) (width 0.25) (layer "B.Cu") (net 17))
 (segment (start 152.825 92.105) (end 150.973299 92.105) (width 0.25) (layer "B.Cu") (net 18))
 (segment (start 154 90.93) (end 152.825 92.105) (width 0.25) (layer "B.Cu") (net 18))
 (segment (start 124.288299 118.79) (end 120.29 118.79) (width 0.25) (layer "B.Cu") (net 18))
 (segment (start 150.973299 92.105) (end 124.288299 118.79) (width 0.25) (layer "B.Cu") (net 18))
 (segment (start 151.46 93.47) (end 124.965 119.965) (width 0.25) (layer "B.Cu") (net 19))
 (segment (start 119.115 119.965) (end 117.75 121.33) (width 0.25) (layer "B.Cu") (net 19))
 (segment (start 124.965 119.965) (end 119.115 119.965) (width 0.25) (layer "B.Cu") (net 19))
 (segment (start 124.42 121.33) (end 120.29 121.33) (width 0.25) (layer "B.Cu") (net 20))
 (segment (start 152.825 94.645) (end 151.105 94.645) (width 0.25) (layer "B.Cu") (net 20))
 (segment (start 154 93.47) (end 152.825 94.645) (width 0.25) (layer "B.Cu") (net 20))
 (segment (start 151.105 94.645) (end 124.42 121.33) (width 0.25) (layer "B.Cu") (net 20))
 (segment (start 151.46 96.01) (end 124.965 122.505) (width 0.25) (layer "B.Cu") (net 21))
 (segment (start 119.115 122.505) (end 117.75 123.87) (width 0.25) (layer "B.Cu") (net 21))
 (segment (start 124.965 122.505) (end 119.115 122.505) (width 0.25) (layer "B.Cu") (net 21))
 (segment (start 152.635 97.375) (end 150.731396 97.375) (width 0.25) (layer "B.Cu") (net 22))
 (segment (start 154 96.01) (end 152.635 97.375) (width 0.25) (layer "B.Cu") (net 22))
 (segment (start 150.731396 97.375) (end 124.236396 123.87) (width 0.25) (layer "B.Cu") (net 22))
 (segment (start 124.236396 123.87) (end 120.29 123.87) (width 0.25) (layer "B.Cu") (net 22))
 (segment (start 151.46 98.55) (end 124.965 125.045) (width 0.25) (layer "B.Cu") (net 23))
 (segment (start 124.965 125.045) (end 119.115 125.045) (width 0.25) (layer "B.Cu") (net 23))
 (segment (start 119.115 125.045) (end 117.75 126.41) (width 0.25) (layer "B.Cu") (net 23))
 (segment (start 154 98.55) (end 152.825 99.725) (width 0.25) (layer "B.Cu") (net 24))
 (segment (start 124.288299 126.41) (end 120.29 126.41) (width 0.25) (layer "B.Cu") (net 24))
 (segment (start 152.825 99.725) (end 150.973299 99.725) (width 0.25) (layer "B.Cu") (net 24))
 (segment (start 150.973299 99.725) (end 124.288299 126.41) (width 0.25) (layer "B.Cu") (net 24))
 (segment (start 124.965 127.585) (end 119.115 127.585) (width 0.25) (layer "B.Cu") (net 25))
 (segment (start 151.46 101.09) (end 124.965 127.585) (width 0.25) (layer "B.Cu") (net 25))
 (segment (start 119.115 127.585) (end 117.75 128.95) (width 0.25) (layer "B.Cu") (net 25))
 (segment (start 154 101.09) (end 152.635 102.455) (width 0.25) (layer "B.Cu") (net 26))
 (segment (start 150.731396 102.455) (end 124.236396 128.95) (width 0.25) (layer "B.Cu") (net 26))
 (segment (start 124.236396 128.95) (end 120.29 128.95) (width 0.25) (layer "B.Cu") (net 26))
 (segment (start 152.635 102.455) (end 150.731396 102.455) (width 0.25) (layer "B.Cu") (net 26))
 (segment (start 139.295 132.665) (end 151.71 145.08) (width 0.25) (layer "F.Cu") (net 27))
 (segment (start 118.925 132.665) (end 139.295 132.665) (width 0.25) (layer "F.Cu") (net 27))
 (segment (start 117.75 131.49) (end 118.925 132.665) (width 0.25) (layer "F.Cu") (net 27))
 (segment (start 120.29 131.49) (end 138.808299 131.49) (width 0.25) (layer "F.Cu") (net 28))
 (segment (start 151.223299 143.905) (end 153.075 143.905) (width 0.25) (layer "F.Cu") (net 28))
 (segment (start 138.808299 131.49) (end 151.223299 143.905) (width 0.25) (layer "F.Cu") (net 28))
 (segment (start 153.075 143.905) (end 154.25 145.08) (width 0.25) (layer "F.Cu") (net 28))
 (segment (start 136.755 135.205) (end 151.71 150.16) (width 0.25) (layer "F.Cu") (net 29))
 (segment (start 117.75 134.03) (end 118.925 135.205) (width 0.25) (layer "F.Cu") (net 29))
 (segment (start 118.925 135.205) (end 136.755 135.205) (width 0.25) (layer "F.Cu") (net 29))
 (segment (start 151.223299 148.985) (end 153.075 148.985) (width 0.25) (layer "F.Cu") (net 30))
 (segment (start 153.075 148.985) (end 154.25 150.16) (width 0.25) (layer "F.Cu") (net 30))
 (segment (start 120.29 134.03) (end 136.268299 134.03) (width 0.25) (layer "F.Cu") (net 30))
 (segment (start 136.268299 134.03) (end 151.223299 148.985) (width 0.25) (layer "F.Cu") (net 30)))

